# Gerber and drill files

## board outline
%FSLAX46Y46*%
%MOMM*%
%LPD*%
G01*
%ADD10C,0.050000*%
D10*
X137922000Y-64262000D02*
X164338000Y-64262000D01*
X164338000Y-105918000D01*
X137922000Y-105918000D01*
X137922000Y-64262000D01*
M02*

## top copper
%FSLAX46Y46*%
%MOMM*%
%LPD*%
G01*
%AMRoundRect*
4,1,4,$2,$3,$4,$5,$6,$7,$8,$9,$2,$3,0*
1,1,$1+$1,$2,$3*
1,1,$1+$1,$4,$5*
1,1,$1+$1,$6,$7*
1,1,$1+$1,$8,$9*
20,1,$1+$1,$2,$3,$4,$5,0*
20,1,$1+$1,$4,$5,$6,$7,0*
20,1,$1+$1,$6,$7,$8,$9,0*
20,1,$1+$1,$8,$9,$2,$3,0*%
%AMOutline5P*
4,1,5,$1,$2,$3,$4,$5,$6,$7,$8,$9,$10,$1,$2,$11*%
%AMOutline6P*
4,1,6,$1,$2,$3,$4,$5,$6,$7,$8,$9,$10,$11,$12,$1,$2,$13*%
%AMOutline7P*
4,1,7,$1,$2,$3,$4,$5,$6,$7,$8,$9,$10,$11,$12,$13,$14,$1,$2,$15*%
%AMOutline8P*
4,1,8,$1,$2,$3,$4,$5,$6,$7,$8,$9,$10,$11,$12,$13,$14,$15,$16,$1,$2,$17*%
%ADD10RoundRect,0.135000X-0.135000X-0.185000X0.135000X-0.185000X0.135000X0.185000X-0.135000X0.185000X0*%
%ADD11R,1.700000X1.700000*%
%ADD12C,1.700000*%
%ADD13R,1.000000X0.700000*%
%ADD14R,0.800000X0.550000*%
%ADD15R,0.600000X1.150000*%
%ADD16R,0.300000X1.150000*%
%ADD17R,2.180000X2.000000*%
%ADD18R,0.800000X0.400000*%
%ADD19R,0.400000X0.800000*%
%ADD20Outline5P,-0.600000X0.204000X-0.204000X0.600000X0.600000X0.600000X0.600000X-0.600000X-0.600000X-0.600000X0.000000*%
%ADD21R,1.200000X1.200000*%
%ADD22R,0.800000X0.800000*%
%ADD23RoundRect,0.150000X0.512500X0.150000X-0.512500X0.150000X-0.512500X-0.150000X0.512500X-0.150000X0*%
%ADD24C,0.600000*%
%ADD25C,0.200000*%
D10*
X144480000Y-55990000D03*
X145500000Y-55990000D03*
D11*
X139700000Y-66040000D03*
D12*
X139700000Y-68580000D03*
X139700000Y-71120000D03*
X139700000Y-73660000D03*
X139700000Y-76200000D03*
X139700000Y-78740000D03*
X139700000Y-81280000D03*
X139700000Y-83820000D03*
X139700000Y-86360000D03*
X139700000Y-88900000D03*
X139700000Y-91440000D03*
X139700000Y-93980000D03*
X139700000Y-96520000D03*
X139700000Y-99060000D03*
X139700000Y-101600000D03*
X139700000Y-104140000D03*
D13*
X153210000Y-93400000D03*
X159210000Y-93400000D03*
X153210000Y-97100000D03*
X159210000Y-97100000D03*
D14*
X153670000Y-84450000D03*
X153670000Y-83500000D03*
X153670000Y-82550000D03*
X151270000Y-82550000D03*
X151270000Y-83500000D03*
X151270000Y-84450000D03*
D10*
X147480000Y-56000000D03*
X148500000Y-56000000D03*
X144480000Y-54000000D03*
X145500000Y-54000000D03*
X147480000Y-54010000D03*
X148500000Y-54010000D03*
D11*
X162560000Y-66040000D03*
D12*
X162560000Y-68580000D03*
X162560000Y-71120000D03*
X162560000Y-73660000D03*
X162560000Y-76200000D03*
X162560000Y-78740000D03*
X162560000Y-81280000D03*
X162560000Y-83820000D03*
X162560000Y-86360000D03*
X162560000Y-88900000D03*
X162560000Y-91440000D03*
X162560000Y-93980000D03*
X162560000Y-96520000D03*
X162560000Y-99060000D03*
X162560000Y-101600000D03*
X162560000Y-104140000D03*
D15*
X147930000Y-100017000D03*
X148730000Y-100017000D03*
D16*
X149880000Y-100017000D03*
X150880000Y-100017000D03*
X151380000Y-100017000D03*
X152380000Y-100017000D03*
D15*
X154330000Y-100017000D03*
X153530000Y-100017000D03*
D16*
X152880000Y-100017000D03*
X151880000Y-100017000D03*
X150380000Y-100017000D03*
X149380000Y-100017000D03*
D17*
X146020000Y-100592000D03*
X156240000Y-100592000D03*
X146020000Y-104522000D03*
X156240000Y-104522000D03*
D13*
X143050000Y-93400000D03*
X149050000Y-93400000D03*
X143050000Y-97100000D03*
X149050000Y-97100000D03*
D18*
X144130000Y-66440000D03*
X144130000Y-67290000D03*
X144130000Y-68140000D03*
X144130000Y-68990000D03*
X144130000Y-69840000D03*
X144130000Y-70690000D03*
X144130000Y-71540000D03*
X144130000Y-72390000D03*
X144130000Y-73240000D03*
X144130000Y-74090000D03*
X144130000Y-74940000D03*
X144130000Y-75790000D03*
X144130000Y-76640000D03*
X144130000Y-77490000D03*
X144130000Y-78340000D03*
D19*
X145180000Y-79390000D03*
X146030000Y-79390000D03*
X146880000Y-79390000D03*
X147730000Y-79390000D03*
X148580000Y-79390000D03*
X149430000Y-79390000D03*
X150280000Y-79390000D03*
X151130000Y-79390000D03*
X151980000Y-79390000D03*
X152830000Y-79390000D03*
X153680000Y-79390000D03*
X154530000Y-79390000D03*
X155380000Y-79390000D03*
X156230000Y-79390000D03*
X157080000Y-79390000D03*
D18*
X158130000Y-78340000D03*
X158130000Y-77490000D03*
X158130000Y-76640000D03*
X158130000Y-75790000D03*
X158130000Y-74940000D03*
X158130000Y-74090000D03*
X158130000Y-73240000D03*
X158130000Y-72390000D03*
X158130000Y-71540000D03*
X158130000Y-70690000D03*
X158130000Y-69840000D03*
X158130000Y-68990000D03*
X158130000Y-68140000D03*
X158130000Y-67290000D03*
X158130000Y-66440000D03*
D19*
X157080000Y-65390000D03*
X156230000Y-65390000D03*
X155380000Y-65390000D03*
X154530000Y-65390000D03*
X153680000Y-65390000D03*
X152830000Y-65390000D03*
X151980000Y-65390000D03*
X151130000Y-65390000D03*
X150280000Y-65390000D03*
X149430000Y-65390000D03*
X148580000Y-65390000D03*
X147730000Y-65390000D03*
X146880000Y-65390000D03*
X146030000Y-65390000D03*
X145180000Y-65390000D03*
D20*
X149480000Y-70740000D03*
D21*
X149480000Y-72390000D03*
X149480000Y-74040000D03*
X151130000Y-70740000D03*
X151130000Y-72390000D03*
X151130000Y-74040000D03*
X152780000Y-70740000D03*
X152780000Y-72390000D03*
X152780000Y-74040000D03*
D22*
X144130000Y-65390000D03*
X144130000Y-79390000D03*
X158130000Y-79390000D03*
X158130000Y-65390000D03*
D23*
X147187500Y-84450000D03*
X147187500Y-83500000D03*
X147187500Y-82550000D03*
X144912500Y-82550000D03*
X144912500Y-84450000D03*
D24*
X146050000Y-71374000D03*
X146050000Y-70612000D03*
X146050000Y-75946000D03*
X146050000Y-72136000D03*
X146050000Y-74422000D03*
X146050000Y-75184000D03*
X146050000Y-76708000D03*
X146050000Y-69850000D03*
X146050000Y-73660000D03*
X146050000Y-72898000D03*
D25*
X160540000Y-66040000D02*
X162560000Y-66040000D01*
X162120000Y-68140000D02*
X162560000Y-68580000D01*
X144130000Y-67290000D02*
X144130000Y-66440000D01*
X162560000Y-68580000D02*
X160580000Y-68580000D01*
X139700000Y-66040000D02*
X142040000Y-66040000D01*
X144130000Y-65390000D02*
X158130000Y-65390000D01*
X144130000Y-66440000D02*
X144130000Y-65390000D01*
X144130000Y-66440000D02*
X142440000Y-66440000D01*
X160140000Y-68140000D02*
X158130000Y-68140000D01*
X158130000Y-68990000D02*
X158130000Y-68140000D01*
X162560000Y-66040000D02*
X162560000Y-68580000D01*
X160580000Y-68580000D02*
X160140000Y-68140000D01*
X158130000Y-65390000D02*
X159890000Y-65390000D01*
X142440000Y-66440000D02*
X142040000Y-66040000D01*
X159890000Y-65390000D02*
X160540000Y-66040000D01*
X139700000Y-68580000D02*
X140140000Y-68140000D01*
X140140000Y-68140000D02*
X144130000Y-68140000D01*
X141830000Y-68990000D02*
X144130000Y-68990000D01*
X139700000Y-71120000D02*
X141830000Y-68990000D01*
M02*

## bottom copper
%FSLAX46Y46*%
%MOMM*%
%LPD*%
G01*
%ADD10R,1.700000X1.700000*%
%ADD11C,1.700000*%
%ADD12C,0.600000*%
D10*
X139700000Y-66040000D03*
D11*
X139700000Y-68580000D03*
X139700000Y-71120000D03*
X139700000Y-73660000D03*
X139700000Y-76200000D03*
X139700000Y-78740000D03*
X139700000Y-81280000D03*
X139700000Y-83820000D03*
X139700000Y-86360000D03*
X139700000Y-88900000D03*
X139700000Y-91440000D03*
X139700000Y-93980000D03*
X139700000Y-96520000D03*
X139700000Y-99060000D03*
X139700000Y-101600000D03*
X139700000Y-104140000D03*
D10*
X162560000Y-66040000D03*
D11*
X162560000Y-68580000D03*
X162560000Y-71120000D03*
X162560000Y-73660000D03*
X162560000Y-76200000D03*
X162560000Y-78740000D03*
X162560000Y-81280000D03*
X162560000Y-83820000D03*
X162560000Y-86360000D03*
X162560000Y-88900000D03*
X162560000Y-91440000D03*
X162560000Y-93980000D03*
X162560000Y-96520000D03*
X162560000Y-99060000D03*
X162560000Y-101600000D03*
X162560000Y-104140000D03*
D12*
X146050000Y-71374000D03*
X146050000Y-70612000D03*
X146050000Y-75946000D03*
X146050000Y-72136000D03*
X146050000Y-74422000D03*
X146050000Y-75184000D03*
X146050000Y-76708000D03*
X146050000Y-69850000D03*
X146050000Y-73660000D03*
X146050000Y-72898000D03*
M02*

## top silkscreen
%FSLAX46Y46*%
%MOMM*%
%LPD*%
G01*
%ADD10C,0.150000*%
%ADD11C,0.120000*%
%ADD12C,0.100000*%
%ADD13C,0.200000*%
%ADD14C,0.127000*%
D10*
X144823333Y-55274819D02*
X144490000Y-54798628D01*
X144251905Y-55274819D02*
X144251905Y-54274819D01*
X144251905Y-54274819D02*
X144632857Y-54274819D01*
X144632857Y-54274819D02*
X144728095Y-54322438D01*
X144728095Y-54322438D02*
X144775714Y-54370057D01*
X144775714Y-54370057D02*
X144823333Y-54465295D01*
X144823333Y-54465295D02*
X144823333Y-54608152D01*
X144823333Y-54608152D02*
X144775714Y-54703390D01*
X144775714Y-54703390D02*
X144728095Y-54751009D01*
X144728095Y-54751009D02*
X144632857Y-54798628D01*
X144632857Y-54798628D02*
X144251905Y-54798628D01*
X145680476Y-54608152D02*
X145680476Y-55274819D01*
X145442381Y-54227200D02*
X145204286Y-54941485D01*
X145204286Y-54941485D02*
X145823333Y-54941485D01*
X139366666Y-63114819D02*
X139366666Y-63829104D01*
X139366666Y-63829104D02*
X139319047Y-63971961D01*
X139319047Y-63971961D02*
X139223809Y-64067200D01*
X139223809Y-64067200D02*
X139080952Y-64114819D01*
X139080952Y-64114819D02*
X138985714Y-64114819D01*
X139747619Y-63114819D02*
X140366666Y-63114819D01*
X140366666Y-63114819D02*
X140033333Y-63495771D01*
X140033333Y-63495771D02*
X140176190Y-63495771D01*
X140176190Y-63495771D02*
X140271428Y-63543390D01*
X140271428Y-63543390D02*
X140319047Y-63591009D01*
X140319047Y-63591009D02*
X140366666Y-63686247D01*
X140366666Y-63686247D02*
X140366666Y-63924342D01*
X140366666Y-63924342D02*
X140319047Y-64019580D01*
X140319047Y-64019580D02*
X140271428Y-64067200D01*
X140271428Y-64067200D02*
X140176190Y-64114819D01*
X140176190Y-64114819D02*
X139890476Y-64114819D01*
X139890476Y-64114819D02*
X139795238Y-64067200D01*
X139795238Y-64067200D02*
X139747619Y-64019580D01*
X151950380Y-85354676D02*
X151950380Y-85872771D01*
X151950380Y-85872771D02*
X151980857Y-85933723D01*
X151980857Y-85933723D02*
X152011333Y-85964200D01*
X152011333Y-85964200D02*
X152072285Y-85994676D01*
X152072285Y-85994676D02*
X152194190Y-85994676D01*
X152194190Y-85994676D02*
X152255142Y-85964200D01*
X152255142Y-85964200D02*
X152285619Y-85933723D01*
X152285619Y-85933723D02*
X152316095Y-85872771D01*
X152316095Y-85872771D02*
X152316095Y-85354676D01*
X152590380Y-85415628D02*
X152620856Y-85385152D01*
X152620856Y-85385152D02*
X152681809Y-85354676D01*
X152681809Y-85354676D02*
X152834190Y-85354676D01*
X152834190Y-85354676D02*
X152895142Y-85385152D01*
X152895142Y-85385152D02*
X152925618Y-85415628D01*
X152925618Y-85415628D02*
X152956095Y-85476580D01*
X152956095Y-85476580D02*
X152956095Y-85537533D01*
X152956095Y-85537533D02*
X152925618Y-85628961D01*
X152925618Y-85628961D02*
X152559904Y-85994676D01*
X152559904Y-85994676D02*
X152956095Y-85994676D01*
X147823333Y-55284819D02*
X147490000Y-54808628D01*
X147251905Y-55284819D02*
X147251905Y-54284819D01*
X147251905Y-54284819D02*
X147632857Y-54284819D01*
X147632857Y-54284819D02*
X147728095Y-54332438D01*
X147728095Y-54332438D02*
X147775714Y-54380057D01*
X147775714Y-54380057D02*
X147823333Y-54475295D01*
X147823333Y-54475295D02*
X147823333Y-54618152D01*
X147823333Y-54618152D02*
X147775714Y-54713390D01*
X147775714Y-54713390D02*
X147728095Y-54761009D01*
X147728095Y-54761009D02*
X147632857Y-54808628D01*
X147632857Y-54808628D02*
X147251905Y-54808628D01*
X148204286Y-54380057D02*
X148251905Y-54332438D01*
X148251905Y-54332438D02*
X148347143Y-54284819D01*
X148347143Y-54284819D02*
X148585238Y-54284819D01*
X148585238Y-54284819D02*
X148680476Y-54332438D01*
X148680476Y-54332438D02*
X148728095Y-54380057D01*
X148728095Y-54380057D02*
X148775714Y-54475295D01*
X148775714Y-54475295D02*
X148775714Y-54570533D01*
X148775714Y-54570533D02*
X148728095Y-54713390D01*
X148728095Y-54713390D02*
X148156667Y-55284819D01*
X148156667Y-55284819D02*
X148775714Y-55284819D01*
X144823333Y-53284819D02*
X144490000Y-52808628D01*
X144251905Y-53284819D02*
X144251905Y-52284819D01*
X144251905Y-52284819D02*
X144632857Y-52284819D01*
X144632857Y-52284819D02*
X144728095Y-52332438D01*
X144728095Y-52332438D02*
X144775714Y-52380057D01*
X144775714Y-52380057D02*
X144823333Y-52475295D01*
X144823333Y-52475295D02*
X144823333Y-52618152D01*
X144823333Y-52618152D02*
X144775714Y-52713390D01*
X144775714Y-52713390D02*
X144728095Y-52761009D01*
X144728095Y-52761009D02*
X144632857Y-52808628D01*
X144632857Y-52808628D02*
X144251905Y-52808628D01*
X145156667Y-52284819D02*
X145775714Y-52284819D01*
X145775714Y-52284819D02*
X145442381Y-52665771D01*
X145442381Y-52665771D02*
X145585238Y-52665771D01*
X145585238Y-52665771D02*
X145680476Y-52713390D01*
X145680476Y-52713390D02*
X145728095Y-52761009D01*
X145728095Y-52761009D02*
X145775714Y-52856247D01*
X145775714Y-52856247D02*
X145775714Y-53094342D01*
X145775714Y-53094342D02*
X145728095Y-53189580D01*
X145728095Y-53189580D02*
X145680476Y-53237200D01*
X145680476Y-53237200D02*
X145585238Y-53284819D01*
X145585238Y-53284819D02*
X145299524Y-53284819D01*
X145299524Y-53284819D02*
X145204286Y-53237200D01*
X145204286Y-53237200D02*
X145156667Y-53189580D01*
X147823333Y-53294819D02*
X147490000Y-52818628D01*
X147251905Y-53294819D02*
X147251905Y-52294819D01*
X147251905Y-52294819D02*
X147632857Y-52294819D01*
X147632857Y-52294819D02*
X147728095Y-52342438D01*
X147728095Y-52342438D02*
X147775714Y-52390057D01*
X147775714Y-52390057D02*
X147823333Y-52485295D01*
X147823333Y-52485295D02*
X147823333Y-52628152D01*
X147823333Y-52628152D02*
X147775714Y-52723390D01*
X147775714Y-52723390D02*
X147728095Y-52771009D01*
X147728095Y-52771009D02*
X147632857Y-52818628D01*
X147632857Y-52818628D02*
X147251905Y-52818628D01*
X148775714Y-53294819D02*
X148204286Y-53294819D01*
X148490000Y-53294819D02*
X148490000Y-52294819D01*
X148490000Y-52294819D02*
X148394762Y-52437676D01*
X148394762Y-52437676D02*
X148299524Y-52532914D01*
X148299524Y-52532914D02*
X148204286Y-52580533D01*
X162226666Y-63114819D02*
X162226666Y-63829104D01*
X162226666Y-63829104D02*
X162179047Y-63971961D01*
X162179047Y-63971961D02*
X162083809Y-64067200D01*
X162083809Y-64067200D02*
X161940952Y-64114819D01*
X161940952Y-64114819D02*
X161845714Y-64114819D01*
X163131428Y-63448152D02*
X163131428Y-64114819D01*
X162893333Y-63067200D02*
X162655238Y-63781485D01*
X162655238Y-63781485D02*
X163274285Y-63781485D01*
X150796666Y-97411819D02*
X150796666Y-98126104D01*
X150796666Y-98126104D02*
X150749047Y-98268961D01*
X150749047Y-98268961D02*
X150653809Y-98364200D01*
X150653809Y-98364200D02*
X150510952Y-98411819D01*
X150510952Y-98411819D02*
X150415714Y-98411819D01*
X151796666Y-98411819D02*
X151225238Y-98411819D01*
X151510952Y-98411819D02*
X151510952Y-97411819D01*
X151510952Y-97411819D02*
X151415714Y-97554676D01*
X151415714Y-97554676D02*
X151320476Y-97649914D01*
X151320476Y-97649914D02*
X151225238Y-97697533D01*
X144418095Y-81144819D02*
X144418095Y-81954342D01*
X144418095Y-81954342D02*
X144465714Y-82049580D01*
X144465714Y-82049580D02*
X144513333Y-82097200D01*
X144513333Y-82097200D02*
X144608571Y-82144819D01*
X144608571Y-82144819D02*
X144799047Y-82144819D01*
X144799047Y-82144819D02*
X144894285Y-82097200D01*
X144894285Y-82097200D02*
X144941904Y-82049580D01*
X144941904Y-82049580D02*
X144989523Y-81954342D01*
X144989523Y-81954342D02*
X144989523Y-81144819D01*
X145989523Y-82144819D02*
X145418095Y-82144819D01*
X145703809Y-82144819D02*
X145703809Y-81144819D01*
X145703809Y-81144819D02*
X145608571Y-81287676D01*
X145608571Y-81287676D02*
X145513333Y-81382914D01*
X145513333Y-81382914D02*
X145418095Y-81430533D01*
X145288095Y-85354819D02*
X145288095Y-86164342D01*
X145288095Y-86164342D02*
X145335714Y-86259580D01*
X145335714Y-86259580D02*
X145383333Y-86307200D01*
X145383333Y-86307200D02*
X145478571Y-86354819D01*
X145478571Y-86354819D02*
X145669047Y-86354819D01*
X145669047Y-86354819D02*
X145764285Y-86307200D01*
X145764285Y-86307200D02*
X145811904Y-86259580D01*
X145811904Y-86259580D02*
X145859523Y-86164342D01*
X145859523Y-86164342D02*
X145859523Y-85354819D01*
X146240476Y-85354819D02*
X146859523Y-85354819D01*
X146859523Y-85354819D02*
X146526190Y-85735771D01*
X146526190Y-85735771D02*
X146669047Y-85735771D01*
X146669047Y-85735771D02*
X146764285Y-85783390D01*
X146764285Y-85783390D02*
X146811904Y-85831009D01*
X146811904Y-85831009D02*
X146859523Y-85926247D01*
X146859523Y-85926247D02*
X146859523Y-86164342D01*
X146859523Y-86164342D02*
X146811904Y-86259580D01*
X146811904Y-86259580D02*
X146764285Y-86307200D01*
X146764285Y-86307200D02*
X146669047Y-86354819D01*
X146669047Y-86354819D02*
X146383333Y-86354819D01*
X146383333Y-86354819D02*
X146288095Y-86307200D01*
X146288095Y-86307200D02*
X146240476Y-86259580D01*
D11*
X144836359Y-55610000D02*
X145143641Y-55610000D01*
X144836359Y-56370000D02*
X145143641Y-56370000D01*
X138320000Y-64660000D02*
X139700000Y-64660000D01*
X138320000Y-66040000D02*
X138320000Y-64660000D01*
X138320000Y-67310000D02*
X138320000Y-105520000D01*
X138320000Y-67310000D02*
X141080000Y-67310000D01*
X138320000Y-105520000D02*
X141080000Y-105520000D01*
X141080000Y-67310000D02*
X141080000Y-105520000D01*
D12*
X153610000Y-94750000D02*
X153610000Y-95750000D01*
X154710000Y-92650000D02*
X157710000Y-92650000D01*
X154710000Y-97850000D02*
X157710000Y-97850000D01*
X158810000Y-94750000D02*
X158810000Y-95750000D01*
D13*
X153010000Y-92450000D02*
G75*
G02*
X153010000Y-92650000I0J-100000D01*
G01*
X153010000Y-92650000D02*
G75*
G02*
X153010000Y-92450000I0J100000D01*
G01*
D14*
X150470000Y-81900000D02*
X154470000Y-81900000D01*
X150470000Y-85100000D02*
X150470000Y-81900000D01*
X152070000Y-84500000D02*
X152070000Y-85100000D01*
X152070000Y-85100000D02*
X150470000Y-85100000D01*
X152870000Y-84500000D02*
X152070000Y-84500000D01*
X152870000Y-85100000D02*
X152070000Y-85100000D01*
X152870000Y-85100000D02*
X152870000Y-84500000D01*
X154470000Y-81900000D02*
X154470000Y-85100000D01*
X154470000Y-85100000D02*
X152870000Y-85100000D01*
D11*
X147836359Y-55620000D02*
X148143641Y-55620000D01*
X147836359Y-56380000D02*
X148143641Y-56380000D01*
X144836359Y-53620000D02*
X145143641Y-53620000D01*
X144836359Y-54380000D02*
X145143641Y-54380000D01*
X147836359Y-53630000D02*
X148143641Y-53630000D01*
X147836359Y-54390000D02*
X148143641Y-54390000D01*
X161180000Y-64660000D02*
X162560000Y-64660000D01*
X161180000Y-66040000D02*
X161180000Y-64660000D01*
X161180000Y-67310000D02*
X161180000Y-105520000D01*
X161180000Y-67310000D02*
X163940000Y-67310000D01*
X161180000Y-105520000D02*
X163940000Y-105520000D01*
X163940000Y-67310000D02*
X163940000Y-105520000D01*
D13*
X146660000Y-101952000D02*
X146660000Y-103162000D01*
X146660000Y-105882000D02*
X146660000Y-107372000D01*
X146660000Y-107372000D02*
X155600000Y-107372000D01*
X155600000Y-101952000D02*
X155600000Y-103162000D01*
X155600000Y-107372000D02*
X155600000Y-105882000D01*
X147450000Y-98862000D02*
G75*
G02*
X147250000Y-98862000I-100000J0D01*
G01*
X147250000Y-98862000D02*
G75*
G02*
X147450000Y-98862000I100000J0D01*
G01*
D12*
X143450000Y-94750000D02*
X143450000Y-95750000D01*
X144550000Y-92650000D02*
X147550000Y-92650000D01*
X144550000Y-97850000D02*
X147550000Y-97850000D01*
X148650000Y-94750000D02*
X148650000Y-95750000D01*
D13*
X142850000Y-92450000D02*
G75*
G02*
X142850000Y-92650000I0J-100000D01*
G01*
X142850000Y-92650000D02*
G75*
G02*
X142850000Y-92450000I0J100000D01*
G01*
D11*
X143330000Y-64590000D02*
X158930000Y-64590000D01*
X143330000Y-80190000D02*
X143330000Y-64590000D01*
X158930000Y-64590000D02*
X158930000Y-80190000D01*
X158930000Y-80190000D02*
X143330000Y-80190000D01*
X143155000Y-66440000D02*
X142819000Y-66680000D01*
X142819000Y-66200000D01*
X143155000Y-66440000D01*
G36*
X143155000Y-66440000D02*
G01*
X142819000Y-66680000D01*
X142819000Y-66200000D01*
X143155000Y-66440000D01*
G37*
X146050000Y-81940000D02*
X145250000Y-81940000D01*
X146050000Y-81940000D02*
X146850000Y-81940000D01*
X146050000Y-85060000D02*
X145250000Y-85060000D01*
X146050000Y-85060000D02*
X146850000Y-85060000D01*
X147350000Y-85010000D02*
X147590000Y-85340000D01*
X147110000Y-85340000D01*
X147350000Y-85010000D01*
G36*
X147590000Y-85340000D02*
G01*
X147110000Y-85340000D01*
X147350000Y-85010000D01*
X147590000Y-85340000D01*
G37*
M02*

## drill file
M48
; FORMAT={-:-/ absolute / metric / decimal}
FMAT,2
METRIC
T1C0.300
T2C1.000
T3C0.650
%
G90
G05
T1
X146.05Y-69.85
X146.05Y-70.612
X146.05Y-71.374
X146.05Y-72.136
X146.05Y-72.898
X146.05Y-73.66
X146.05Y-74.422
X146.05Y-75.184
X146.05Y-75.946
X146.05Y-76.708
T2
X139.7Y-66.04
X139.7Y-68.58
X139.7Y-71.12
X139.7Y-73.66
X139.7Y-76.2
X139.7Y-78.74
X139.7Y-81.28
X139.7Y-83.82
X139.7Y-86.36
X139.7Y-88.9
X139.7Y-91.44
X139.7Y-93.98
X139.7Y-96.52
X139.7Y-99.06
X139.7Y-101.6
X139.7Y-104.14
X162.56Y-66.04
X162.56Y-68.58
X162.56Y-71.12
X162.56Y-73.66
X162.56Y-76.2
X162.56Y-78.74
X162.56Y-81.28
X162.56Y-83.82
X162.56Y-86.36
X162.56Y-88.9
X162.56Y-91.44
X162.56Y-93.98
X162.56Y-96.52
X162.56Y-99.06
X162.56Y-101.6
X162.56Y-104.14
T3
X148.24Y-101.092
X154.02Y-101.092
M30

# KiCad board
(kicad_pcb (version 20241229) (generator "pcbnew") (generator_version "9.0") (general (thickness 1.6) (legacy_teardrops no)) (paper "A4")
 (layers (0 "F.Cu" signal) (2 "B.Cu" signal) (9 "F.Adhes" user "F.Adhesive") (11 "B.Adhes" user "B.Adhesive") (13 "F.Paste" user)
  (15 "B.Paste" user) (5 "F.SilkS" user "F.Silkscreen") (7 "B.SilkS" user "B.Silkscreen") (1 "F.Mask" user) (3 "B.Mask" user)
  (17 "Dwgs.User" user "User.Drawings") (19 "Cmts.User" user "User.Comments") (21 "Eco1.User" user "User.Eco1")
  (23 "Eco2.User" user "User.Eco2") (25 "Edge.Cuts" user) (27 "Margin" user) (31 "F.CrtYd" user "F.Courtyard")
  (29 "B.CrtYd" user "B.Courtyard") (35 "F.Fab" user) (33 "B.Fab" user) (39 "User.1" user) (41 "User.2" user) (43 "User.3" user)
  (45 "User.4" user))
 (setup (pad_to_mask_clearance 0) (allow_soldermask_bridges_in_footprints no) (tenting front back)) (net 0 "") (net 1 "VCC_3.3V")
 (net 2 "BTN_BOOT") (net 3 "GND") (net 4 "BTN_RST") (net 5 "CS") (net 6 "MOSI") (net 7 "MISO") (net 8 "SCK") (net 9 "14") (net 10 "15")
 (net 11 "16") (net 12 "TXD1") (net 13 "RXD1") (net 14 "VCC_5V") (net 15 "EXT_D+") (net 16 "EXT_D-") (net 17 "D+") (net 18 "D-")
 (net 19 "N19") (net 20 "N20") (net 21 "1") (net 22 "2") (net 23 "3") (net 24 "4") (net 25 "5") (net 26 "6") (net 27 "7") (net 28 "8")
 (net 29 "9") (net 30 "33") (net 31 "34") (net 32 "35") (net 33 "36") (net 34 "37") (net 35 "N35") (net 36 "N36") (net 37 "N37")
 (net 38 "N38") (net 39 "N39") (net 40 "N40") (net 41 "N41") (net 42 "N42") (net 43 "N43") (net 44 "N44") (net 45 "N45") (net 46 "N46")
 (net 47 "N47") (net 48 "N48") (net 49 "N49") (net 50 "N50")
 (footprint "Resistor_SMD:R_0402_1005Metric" (layer "F.Cu") (at 144.99 55.99)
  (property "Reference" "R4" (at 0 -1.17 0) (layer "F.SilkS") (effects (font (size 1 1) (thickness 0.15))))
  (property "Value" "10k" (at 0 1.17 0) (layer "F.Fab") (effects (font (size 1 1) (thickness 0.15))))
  (fp_line (start -0.153641 -0.38) (end 0.153641 -0.38) (stroke (width 0.12) (type solid)) (layer "F.SilkS"))
  (fp_line (start -0.153641 0.38) (end 0.153641 0.38) (stroke (width 0.12) (type solid)) (layer "F.SilkS"))
  (pad "1" smd roundrect (at -0.51 0) (size 0.54 0.64) (layers "F.Cu" "F.Mask" "F.Paste") (roundrect_rratio 0.25) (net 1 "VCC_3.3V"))
  (pad "2" smd roundrect (at 0.51 0) (size 0.54 0.64) (layers "F.Cu" "F.Mask" "F.Paste") (roundrect_rratio 0.25) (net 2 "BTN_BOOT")))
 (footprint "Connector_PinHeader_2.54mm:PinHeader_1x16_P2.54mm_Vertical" (layer "F.Cu") (at 139.7 66.04)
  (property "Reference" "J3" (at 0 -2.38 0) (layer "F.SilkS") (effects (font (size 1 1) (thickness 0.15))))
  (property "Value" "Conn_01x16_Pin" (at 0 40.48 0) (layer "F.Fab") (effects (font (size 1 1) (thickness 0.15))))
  (fp_line (start -1.38 -1.38) (end 0 -1.38) (stroke (width 0.12) (type solid)) (layer "F.SilkS"))
  (fp_line (start -1.38 0) (end -1.38 -1.38) (stroke (width 0.12) (type solid)) (layer "F.SilkS"))
  (fp_line (start -1.38 1.27) (end -1.38 39.48) (stroke (width 0.12) (type solid)) (layer "F.SilkS"))
  (fp_line (start -1.38 1.27) (end 1.38 1.27) (stroke (width 0.12) (type solid)) (layer "F.SilkS"))
  (fp_line (start -1.38 39.48) (end 1.38 39.48) (stroke (width 0.12) (type solid)) (layer "F.SilkS"))
  (fp_line (start 1.38 1.27) (end 1.38 39.48) (stroke (width 0.12) (type solid)) (layer "F.SilkS"))
  (pad "1" thru_hole rect (at 0 0) (size 1.7 1.7) (drill 1) (layers "*.Cu" "*.Mask") (remove_unused_layers no) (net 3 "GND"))
  (pad "2" thru_hole circle (at 0 2.54) (size 1.7 1.7) (drill 1) (layers "*.Cu" "*.Mask") (remove_unused_layers no) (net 1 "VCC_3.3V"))
  (pad "3" thru_hole circle (at 0 5.08) (size 1.7 1.7) (drill 1) (layers "*.Cu" "*.Mask") (remove_unused_layers no) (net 2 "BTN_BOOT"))
  (pad "4" thru_hole circle (at 0 7.62) (size 1.7 1.7) (drill 1) (layers "*.Cu" "*.Mask") (remove_unused_layers no) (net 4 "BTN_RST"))
  (pad "5" thru_hole circle (at 0 10.16) (size 1.7 1.7) (drill 1) (layers "*.Cu" "*.Mask") (remove_unused_layers no) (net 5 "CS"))
  (pad "6" thru_hole circle (at 0 12.7) (size 1.7 1.7) (drill 1) (layers "*.Cu" "*.Mask") (remove_unused_layers no) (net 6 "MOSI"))
  (pad "7" thru_hole circle (at 0 15.24) (size 1.7 1.7) (drill 1) (layers "*.Cu" "*.Mask") (remove_unused_layers no) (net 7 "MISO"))
  (pad "8" thru_hole circle (at 0 17.78) (size 1.7 1.7) (drill 1) (layers "*.Cu" "*.Mask") (remove_unused_layers no) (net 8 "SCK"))
  (pad "9" thru_hole circle (at 0 20.32) (size 1.7 1.7) (drill 1) (layers "*.Cu" "*.Mask") (remove_unused_layers no) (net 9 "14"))
  (pad "10" thru_hole circle (at 0 22.86) (size 1.7 1.7) (drill 1) (layers "*.Cu" "*.Mask") (remove_unused_layers no) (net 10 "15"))
  (pad "11" thru_hole circle (at 0 25.4) (size 1.7 1.7) (drill 1) (layers "*.Cu" "*.Mask") (remove_unused_layers no) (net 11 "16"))
  (pad "12" thru_hole circle (at 0 27.94) (size 1.7 1.7) (drill 1) (layers "*.Cu" "*.Mask") (remove_unused_layers no) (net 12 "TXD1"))
  (pad "13" thru_hole circle (at 0 30.48) (size 1.7 1.7) (drill 1) (layers "*.Cu" "*.Mask") (remove_unused_layers no) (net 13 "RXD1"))
  (pad "14" thru_hole circle (at 0 33.02) (size 1.7 1.7) (drill 1) (layers "*.Cu" "*.Mask") (remove_unused_layers no) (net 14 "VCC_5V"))
  (pad "15" thru_hole circle (at 0 35.56) (size 1.7 1.7) (drill 1) (layers "*.Cu" "*.Mask") (remove_unused_layers no) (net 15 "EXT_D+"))
  (pad "16" thru_hole circle (at 0 38.1) (size 1.7 1.7) (drill 1) (layers "*.Cu" "*.Mask") (remove_unused_layers no) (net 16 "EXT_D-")))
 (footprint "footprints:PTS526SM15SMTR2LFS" (layer "F.Cu") (at 156.21 95.25)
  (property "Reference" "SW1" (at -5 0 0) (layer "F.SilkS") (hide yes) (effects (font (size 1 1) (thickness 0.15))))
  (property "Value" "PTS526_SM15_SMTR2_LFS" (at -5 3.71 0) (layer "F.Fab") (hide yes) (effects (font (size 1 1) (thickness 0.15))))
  (fp_line (start -2.6 -0.5) (end -2.6 0.5) (stroke (width 0.1) (type solid)) (layer "F.SilkS"))
  (fp_line (start -1.5 -2.6) (end 1.5 -2.6) (stroke (width 0.1) (type solid)) (layer "F.SilkS"))
  (fp_line (start -1.5 2.6) (end 1.5 2.6) (stroke (width 0.1) (type solid)) (layer "F.SilkS"))
  (fp_line (start 2.6 -0.5) (end 2.6 0.5) (stroke (width 0.1) (type solid)) (layer "F.SilkS"))
  (fp_arc (start -3.2 -2.8) (mid -3.1 -2.7) (end -3.2 -2.6) (stroke (width 0.2) (type solid)) (layer "F.SilkS"))
  (fp_arc (start -3.2 -2.6) (mid -3.3 -2.7) (end -3.2 -2.8) (stroke (width 0.2) (type solid)) (layer "F.SilkS"))
  (pad "1" smd rect (at -3 -1.85) (size 1 0.7) (layers "F.Cu" "F.Mask" "F.Paste") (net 3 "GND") (solder_mask_margin 0.102))
  (pad "2" smd rect (at 3 -1.85) (size 1 0.7) (layers "F.Cu" "F.Mask" "F.Paste") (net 3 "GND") (solder_mask_margin 0.102))
  (pad "3" smd rect (at -3 1.85) (size 1 0.7) (layers "F.Cu" "F.Mask" "F.Paste") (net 4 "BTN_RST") (solder_mask_margin 0.102))
  (pad "4" smd rect (at 3 1.85) (size 1 0.7) (layers "F.Cu" "F.Mask" "F.Paste") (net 4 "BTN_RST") (solder_mask_margin 0.102)))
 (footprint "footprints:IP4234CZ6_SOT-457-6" (layer "F.Cu") (at 152.47 83.5 180)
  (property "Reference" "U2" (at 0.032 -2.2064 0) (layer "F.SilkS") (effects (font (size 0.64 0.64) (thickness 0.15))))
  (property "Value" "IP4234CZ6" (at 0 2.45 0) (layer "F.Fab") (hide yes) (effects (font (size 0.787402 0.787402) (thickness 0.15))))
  (fp_line (start 2 1.6) (end -2 1.6) (stroke (width 0.127) (type solid)) (layer "F.SilkS"))
  (fp_line (start 2 -1.6) (end 2 1.6) (stroke (width 0.127) (type solid)) (layer "F.SilkS"))
  (fp_line (start 0.4 -1) (end 0.4 -1.6) (stroke (width 0.127) (type solid)) (layer "F.SilkS"))
  (fp_line (start 0.4 -1.6) (end 2 -1.6) (stroke (width 0.127) (type solid)) (layer "F.SilkS"))
  (fp_line (start -0.4 -1) (end 0.4 -1) (stroke (width 0.127) (type solid)) (layer "F.SilkS"))
  (fp_line (start -0.4 -1.6) (end 0.4 -1.6) (stroke (width 0.127) (type solid)) (layer "F.SilkS"))
  (fp_line (start -0.4 -1.6) (end -0.4 -1) (stroke (width 0.127) (type solid)) (layer "F.SilkS"))
  (fp_line (start -2 1.6) (end -2 -1.6) (stroke (width 0.127) (type solid)) (layer "F.SilkS"))
  (fp_line (start -2 -1.6) (end -0.4 -1.6) (stroke (width 0.127) (type solid)) (layer "F.SilkS"))
  (pad "1" smd rect (at -1.2 -0.95 180) (size 0.8 0.55) (layers "F.Cu" "F.Mask" "F.Paste") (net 15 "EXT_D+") (solder_mask_margin 0.102))
  (pad "2" smd rect (at -1.2 0 180) (size 0.8 0.55) (layers "F.Cu" "F.Mask" "F.Paste") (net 3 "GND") (solder_mask_margin 0.102))
  (pad "3" smd rect (at -1.2 0.95 180) (size 0.8 0.55) (layers "F.Cu" "F.Mask" "F.Paste") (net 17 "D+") (solder_mask_margin 0.102))
  (pad "4" smd rect (at 1.2 0.95 180) (size 0.8 0.55) (layers "F.Cu" "F.Mask" "F.Paste") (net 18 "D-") (solder_mask_margin 0.102))
  (pad "5" smd rect (at 1.2 0 180) (size 0.8 0.55) (layers "F.Cu" "F.Mask" "F.Paste") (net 14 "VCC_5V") (solder_mask_margin 0.102))
  (pad "6" smd rect (at 1.2 -0.95 180) (size 0.8 0.55) (layers "F.Cu" "F.Mask" "F.Paste") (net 16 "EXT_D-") (solder_mask_margin 0.102)))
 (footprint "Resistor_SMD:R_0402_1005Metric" (layer "F.Cu") (at 147.99 56)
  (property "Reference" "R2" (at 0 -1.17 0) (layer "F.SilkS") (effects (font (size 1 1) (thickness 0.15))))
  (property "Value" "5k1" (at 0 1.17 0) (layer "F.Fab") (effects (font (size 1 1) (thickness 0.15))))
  (fp_line (start -0.153641 -0.38) (end 0.153641 -0.38) (stroke (width 0.12) (type solid)) (layer "F.SilkS"))
  (fp_line (start -0.153641 0.38) (end 0.153641 0.38) (stroke (width 0.12) (type solid)) (layer "F.SilkS"))
  (pad "1" smd roundrect (at -0.51 0) (size 0.54 0.64) (layers "F.Cu" "F.Mask" "F.Paste") (roundrect_rratio 0.25) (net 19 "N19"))
  (pad "2" smd roundrect (at 0.51 0) (size 0.54 0.64) (layers "F.Cu" "F.Mask" "F.Paste") (roundrect_rratio 0.25) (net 3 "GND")))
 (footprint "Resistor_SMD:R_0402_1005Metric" (layer "F.Cu") (at 144.99 54)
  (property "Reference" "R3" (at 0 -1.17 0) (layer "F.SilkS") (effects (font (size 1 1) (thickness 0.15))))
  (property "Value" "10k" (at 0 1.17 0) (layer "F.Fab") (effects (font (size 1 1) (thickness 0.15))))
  (fp_line (start -0.153641 -0.38) (end 0.153641 -0.38) (stroke (width 0.12) (type solid)) (layer "F.SilkS"))
  (fp_line (start -0.153641 0.38) (end 0.153641 0.38) (stroke (width 0.12) (type solid)) (layer "F.SilkS"))
  (pad "1" smd roundrect (at -0.51 0) (size 0.54 0.64) (layers "F.Cu" "F.Mask" "F.Paste") (roundrect_rratio 0.25) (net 1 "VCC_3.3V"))
  (pad "2" smd roundrect (at 0.51 0) (size 0.54 0.64) (layers "F.Cu" "F.Mask" "F.Paste") (roundrect_rratio 0.25) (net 4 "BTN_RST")))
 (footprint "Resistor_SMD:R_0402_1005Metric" (layer "F.Cu") (at 147.99 54.01)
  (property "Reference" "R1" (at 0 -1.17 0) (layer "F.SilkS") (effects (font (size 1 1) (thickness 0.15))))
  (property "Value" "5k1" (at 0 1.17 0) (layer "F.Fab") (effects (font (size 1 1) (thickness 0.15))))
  (fp_line (start -0.153641 -0.38) (end 0.153641 -0.38) (stroke (width 0.12) (type solid)) (layer "F.SilkS"))
  (fp_line (start -0.153641 0.38) (end 0.153641 0.38) (stroke (width 0.12) (type solid)) (layer "F.SilkS"))
  (pad "1" smd roundrect (at -0.51 0) (size 0.54 0.64) (layers "F.Cu" "F.Mask" "F.Paste") (roundrect_rratio 0.25) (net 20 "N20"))
  (pad "2" smd roundrect (at 0.51 0) (size 0.54 0.64) (layers "F.Cu" "F.Mask" "F.Paste") (roundrect_rratio 0.25) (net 3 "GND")))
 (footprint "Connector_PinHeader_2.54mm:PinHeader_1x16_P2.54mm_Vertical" (layer "F.Cu") (at 162.56 66.04)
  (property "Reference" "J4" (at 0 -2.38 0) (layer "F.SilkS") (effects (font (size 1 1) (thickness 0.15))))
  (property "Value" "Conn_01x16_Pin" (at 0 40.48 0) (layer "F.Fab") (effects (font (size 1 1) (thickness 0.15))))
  (fp_line (start -1.38 -1.38) (end 0 -1.38) (stroke (width 0.12) (type solid)) (layer "F.SilkS"))
  (fp_line (start -1.38 0) (end -1.38 -1.38) (stroke (width 0.12) (type solid)) (layer "F.SilkS"))
  (fp_line (start -1.38 1.27) (end -1.38 39.48) (stroke (width 0.12) (type solid)) (layer "F.SilkS"))
  (fp_line (start -1.38 1.27) (end 1.38 1.27) (stroke (width 0.12) (type solid)) (layer "F.SilkS"))
  (fp_line (start -1.38 39.48) (end 1.38 39.48) (stroke (width 0.12) (type solid)) (layer "F.SilkS"))
  (fp_line (start 1.38 1.27) (end 1.38 39.48) (stroke (width 0.12) (type solid)) (layer "F.SilkS"))
  (pad "1" thru_hole rect (at 0 0) (size 1.7 1.7) (drill 1) (layers "*.Cu" "*.Mask") (remove_unused_layers no) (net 3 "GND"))
  (pad "2" thru_hole circle (at 0 2.54) (size 1.7 1.7) (drill 1) (layers "*.Cu" "*.Mask") (remove_unused_layers no) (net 3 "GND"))
  (pad "3" thru_hole circle (at 0 5.08) (size 1.7 1.7) (drill 1) (layers "*.Cu" "*.Mask") (remove_unused_layers no) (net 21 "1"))
  (pad "4" thru_hole circle (at 0 7.62) (size 1.7 1.7) (drill 1) (layers "*.Cu" "*.Mask") (remove_unused_layers no) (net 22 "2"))
  (pad "5" thru_hole circle (at 0 10.16) (size 1.7 1.7) (drill 1) (layers "*.Cu" "*.Mask") (remove_unused_layers no) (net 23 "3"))
  (pad "6" thru_hole circle (at 0 12.7) (size 1.7 1.7) (drill 1) (layers "*.Cu" "*.Mask") (remove_unused_layers no) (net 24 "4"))
  (pad "7" thru_hole circle (at 0 15.24) (size 1.7 1.7) (drill 1) (layers "*.Cu" "*.Mask") (remove_unused_layers no) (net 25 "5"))
  (pad "8" thru_hole circle (at 0 17.78) (size 1.7 1.7) (drill 1) (layers "*.Cu" "*.Mask") (remove_unused_layers no) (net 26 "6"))
  (pad "9" thru_hole circle (at 0 20.32) (size 1.7 1.7) (drill 1) (layers "*.Cu" "*.Mask") (remove_unused_layers no) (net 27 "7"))
  (pad "10" thru_hole circle (at 0 22.86) (size 1.7 1.7) (drill 1) (layers "*.Cu" "*.Mask") (remove_unused_layers no) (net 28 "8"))
  (pad "11" thru_hole circle (at 0 25.4) (size 1.7 1.7) (drill 1) (layers "*.Cu" "*.Mask") (remove_unused_layers no) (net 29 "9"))
  (pad "12" thru_hole circle (at 0 27.94) (size 1.7 1.7) (drill 1) (layers "*.Cu" "*.Mask") (remove_unused_layers no) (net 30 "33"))
  (pad "13" thru_hole circle (at 0 30.48) (size 1.7 1.7) (drill 1) (layers "*.Cu" "*.Mask") (remove_unused_layers no) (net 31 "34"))
  (pad "14" thru_hole circle (at 0 33.02) (size 1.7 1.7) (drill 1) (layers "*.Cu" "*.Mask") (remove_unused_layers no) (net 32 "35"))
  (pad "15" thru_hole circle (at 0 35.56) (size 1.7 1.7) (drill 1) (layers "*.Cu" "*.Mask") (remove_unused_layers no) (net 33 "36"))
  (pad "16" thru_hole circle (at 0 38.1) (size 1.7 1.7) (drill 1) (layers "*.Cu" "*.Mask") (remove_unused_layers no) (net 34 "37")))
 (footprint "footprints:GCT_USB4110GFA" (layer "F.Cu") (at 151.13 101.092)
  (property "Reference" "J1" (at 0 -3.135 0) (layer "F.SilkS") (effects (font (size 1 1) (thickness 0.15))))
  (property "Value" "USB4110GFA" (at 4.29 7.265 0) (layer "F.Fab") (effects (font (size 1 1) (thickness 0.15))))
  (fp_line (start -4.47 0.86) (end -4.47 2.07) (stroke (width 0.2) (type solid)) (layer "F.SilkS"))
  (fp_line (start -4.47 4.79) (end -4.47 6.28) (stroke (width 0.2) (type solid)) (layer "F.SilkS"))
  (fp_line (start -4.47 6.28) (end 4.47 6.28) (stroke (width 0.2) (type solid)) (layer "F.SilkS"))
  (fp_line (start 4.47 0.86) (end 4.47 2.07) (stroke (width 0.2) (type solid)) (layer "F.SilkS"))
  (fp_line (start 4.47 6.28) (end 4.47 4.79) (stroke (width 0.2) (type solid)) (layer "F.SilkS"))
  (fp_circle (center -3.78 -2.23) (end -3.68 -2.23) (stroke (width 0.2) (type solid)) (fill no) (layer "F.SilkS"))
  (pad "" np_thru_hole circle (at -2.89 0) (size 0.65 0.65) (drill 0.65) (layers "*.Cu" "*.Mask"))
  (pad "" np_thru_hole circle (at 2.89 0) (size 0.65 0.65) (drill 0.65) (layers "*.Cu" "*.Mask"))
  (pad "A1/B12" smd rect (at -3.2 -1.075) (size 0.6 1.15) (layers "F.Cu" "F.Mask" "F.Paste") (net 3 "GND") (solder_mask_margin 0.102))
  (pad "A4/B9" smd rect (at -2.4 -1.075) (size 0.6 1.15) (layers "F.Cu" "F.Mask" "F.Paste") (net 14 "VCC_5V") (solder_mask_margin 0.102))
  (pad "A5" smd rect (at -1.25 -1.075) (size 0.3 1.15) (layers "F.Cu" "F.Mask" "F.Paste") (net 20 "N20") (solder_mask_margin 0.102))
  (pad "A6" smd rect (at -0.25 -1.075) (size 0.3 1.15) (layers "F.Cu" "F.Mask" "F.Paste") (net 15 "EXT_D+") (solder_mask_margin 0.102))
  (pad "A7" smd rect (at 0.25 -1.075) (size 0.3 1.15) (layers "F.Cu" "F.Mask" "F.Paste") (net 16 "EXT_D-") (solder_mask_margin 0.102))
  (pad "A8" smd rect (at 1.25 -1.075) (size 0.3 1.15) (layers "F.Cu" "F.Mask" "F.Paste") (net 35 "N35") (solder_mask_margin 0.102))
  (pad "B1/A12" smd rect (at 3.2 -1.075) (size 0.6 1.15) (layers "F.Cu" "F.Mask" "F.Paste") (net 3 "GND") (solder_mask_margin 0.102))
  (pad "B4/A9" smd rect (at 2.4 -1.075) (size 0.6 1.15) (layers "F.Cu" "F.Mask" "F.Paste") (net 14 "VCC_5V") (solder_mask_margin 0.102))
  (pad "B5" smd rect (at 1.75 -1.075) (size 0.3 1.15) (layers "F.Cu" "F.Mask" "F.Paste") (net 19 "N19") (solder_mask_margin 0.102))
  (pad "B6" smd rect (at 0.75 -1.075) (size 0.3 1.15) (layers "F.Cu" "F.Mask" "F.Paste") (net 15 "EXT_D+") (solder_mask_margin 0.102))
  (pad "B7" smd rect (at -0.75 -1.075) (size 0.3 1.15) (layers "F.Cu" "F.Mask" "F.Paste") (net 16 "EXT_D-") (solder_mask_margin 0.102))
  (pad "B8" smd rect (at -1.75 -1.075) (size 0.3 1.15) (layers "F.Cu" "F.Mask" "F.Paste") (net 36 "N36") (solder_mask_margin 0.102))
  (pad "S1" smd rect (at -5.11 -0.5) (size 2.18 2) (layers "F.Cu" "F.Mask" "F.Paste") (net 3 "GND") (solder_mask_margin 0.102))
  (pad "S2" smd rect (at 5.11 -0.5) (size 2.18 2) (layers "F.Cu" "F.Mask" "F.Paste") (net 3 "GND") (solder_mask_margin 0.102))
  (pad "S3" smd rect (at -5.11 3.43) (size 2.18 2) (layers "F.Cu" "F.Mask" "F.Paste") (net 3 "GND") (solder_mask_margin 0.102))
  (pad "S4" smd rect (at 5.11 3.43) (size 2.18 2) (layers "F.Cu" "F.Mask" "F.Paste") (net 3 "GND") (solder_mask_margin 0.102)))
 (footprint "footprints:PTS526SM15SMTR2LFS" (layer "F.Cu") (at 146.05 95.25)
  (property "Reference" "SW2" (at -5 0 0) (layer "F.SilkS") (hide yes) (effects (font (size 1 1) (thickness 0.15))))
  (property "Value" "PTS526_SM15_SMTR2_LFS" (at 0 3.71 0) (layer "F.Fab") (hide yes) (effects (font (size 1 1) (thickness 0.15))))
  (fp_line (start -2.6 -0.5) (end -2.6 0.5) (stroke (width 0.1) (type solid)) (layer "F.SilkS"))
  (fp_line (start -1.5 -2.6) (end 1.5 -2.6) (stroke (width 0.1) (type solid)) (layer "F.SilkS"))
  (fp_line (start -1.5 2.6) (end 1.5 2.6) (stroke (width 0.1) (type solid)) (layer "F.SilkS"))
  (fp_line (start 2.6 -0.5) (end 2.6 0.5) (stroke (width 0.1) (type solid)) (layer "F.SilkS"))
  (fp_arc (start -3.2 -2.8) (mid -3.1 -2.7) (end -3.2 -2.6) (stroke (width 0.2) (type solid)) (layer "F.SilkS"))
  (fp_arc (start -3.2 -2.6) (mid -3.3 -2.7) (end -3.2 -2.8) (stroke (width 0.2) (type solid)) (layer "F.SilkS"))
  (pad "1" smd rect (at -3 -1.85) (size 1 0.7) (layers "F.Cu" "F.Mask" "F.Paste") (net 3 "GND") (solder_mask_margin 0.102))
  (pad "2" smd rect (at 3 -1.85) (size 1 0.7) (layers "F.Cu" "F.Mask" "F.Paste") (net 3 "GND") (solder_mask_margin 0.102))
  (pad "3" smd rect (at -3 1.85) (size 1 0.7) (layers "F.Cu" "F.Mask" "F.Paste") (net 2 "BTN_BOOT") (solder_mask_margin 0.102))
  (pad "4" smd rect (at 3 1.85) (size 1 0.7) (layers "F.Cu" "F.Mask" "F.Paste") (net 2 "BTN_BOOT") (solder_mask_margin 0.102)))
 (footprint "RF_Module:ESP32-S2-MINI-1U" (layer "F.Cu") (at 151.13 72.39)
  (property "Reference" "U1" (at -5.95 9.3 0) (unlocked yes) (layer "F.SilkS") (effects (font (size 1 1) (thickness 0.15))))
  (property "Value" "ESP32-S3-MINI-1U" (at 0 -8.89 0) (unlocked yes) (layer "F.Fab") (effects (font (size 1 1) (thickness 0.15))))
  (fp_line (start -7.8 -7.8) (end 7.8 -7.8) (stroke (width 0.12) (type solid)) (layer "F.SilkS"))
  (fp_line (start -7.8 7.8) (end -7.8 -7.8) (stroke (width 0.12) (type solid)) (layer "F.SilkS"))
  (fp_line (start 7.8 -7.8) (end 7.8 7.8) (stroke (width 0.12) (type solid)) (layer "F.SilkS"))
  (fp_line (start 7.8 7.8) (end -7.8 7.8) (stroke (width 0.12) (type solid)) (layer "F.SilkS"))
  (fp_poly
   (pts (xy -7.975 -5.95) (xy -8.311 -5.71) (xy -8.311 -6.19) (xy -7.975 -5.95)) (stroke (width 0.12) (type solid)) (fill yes)
   (layer "F.SilkS"))
  (pad "1" smd rect (at -7 -5.95) (size 0.8 0.4) (layers "F.Cu" "F.Mask" "F.Paste") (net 3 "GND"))
  (pad "2" smd rect (at -7 -5.1) (size 0.8 0.4) (layers "F.Cu" "F.Mask" "F.Paste") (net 3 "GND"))
  (pad "3" smd rect (at -7 -4.25) (size 0.8 0.4) (layers "F.Cu" "F.Mask" "F.Paste") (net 1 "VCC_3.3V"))
  (pad "4" smd rect (at -7 -3.4) (size 0.8 0.4) (layers "F.Cu" "F.Mask" "F.Paste") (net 2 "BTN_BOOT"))
  (pad "5" smd rect (at -7 -2.55) (size 0.8 0.4) (layers "F.Cu" "F.Mask" "F.Paste") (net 21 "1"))
  (pad "6" smd rect (at -7 -1.7) (size 0.8 0.4) (layers "F.Cu" "F.Mask" "F.Paste") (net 22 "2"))
  (pad "7" smd rect (at -7 -0.85) (size 0.8 0.4) (layers "F.Cu" "F.Mask" "F.Paste") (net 23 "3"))
  (pad "8" smd rect (at -7 0) (size 0.8 0.4) (layers "F.Cu" "F.Mask" "F.Paste") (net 24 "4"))
  (pad "9" smd rect (at -7 0.85) (size 0.8 0.4) (layers "F.Cu" "F.Mask" "F.Paste") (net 25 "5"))
  (pad "10" smd rect (at -7 1.7) (size 0.8 0.4) (layers "F.Cu" "F.Mask" "F.Paste") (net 26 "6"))
  (pad "11" smd rect (at -7 2.55) (size 0.8 0.4) (layers "F.Cu" "F.Mask" "F.Paste") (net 27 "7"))
  (pad "12" smd rect (at -7 3.4) (size 0.8 0.4) (layers "F.Cu" "F.Mask" "F.Paste") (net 28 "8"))
  (pad "13" smd rect (at -7 4.25) (size 0.8 0.4) (layers "F.Cu" "F.Mask" "F.Paste") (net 29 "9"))
  (pad "14" smd rect (at -7 5.1) (size 0.8 0.4) (layers "F.Cu" "F.Mask" "F.Paste") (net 5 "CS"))
  (pad "15" smd rect (at -7 5.95) (size 0.8 0.4) (layers "F.Cu" "F.Mask" "F.Paste") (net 6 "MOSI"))
  (pad "16" smd rect (at -5.95 7 90) (size 0.8 0.4) (layers "F.Cu" "F.Mask" "F.Paste") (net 7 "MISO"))
  (pad "17" smd rect (at -5.1 7 90) (size 0.8 0.4) (layers "F.Cu" "F.Mask" "F.Paste") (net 8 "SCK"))
  (pad "18" smd rect (at -4.25 7 90) (size 0.8 0.4) (layers "F.Cu" "F.Mask" "F.Paste") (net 9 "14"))
  (pad "19" smd rect (at -3.4 7 90) (size 0.8 0.4) (layers "F.Cu" "F.Mask" "F.Paste") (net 10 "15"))
  (pad "20" smd rect (at -2.55 7 90) (size 0.8 0.4) (layers "F.Cu" "F.Mask" "F.Paste") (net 11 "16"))
  (pad "21" smd rect (at -1.7 7 90) (size 0.8 0.4) (layers "F.Cu" "F.Mask" "F.Paste") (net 12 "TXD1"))
  (pad "22" smd rect (at -0.85 7 90) (size 0.8 0.4) (layers "F.Cu" "F.Mask" "F.Paste") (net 13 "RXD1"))
  (pad "23" smd rect (at 0 7 90) (size 0.8 0.4) (layers "F.Cu" "F.Mask" "F.Paste") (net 18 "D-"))
  (pad "24" smd rect (at 0.85 7 90) (size 0.8 0.4) (layers "F.Cu" "F.Mask" "F.Paste") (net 17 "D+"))
  (pad "25" smd rect (at 1.7 7 90) (size 0.8 0.4) (layers "F.Cu" "F.Mask" "F.Paste") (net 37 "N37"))
  (pad "26" smd rect (at 2.55 7 90) (size 0.8 0.4) (layers "F.Cu" "F.Mask" "F.Paste") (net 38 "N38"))
  (pad "27" smd rect (at 3.4 7 90) (size 0.8 0.4) (layers "F.Cu" "F.Mask" "F.Paste") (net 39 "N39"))
  (pad "28" smd rect (at 4.25 7 90) (size 0.8 0.4) (layers "F.Cu" "F.Mask" "F.Paste") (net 30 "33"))
  (pad "29" smd rect (at 5.1 7 90) (size 0.8 0.4) (layers "F.Cu" "F.Mask" "F.Paste") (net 31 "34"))
  (pad "30" smd rect (at 5.95 7 90) (size 0.8 0.4) (layers "F.Cu" "F.Mask" "F.Paste") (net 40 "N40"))
  (pad "31" smd rect (at 7 5.95) (size 0.8 0.4) (layers "F.Cu" "F.Mask" "F.Paste") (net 32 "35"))
  (pad "32" smd rect (at 7 5.1) (size 0.8 0.4) (layers "F.Cu" "F.Mask" "F.Paste") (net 33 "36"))
  (pad "33" smd rect (at 7 4.25) (size 0.8 0.4) (layers "F.Cu" "F.Mask" "F.Paste") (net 34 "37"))
  (pad "34" smd rect (at 7 3.4) (size 0.8 0.4) (layers "F.Cu" "F.Mask" "F.Paste") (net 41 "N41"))
  (pad "35" smd rect (at 7 2.55) (size 0.8 0.4) (layers "F.Cu" "F.Mask" "F.Paste") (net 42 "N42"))
  (pad "36" smd rect (at 7 1.7) (size 0.8 0.4) (layers "F.Cu" "F.Mask" "F.Paste") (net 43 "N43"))
  (pad "37" smd rect (at 7 0.85) (size 0.8 0.4) (layers "F.Cu" "F.Mask" "F.Paste") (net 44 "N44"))
  (pad "38" smd rect (at 7 0) (size 0.8 0.4) (layers "F.Cu" "F.Mask" "F.Paste") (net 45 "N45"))
  (pad "39" smd rect (at 7 -0.85) (size 0.8 0.4) (layers "F.Cu" "F.Mask" "F.Paste") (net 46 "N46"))
  (pad "40" smd rect (at 7 -1.7) (size 0.8 0.4) (layers "F.Cu" "F.Mask" "F.Paste") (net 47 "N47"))
  (pad "41" smd rect (at 7 -2.55) (size 0.8 0.4) (layers "F.Cu" "F.Mask" "F.Paste") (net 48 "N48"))
  (pad "42" smd rect (at 7 -3.4) (size 0.8 0.4) (layers "F.Cu" "F.Mask" "F.Paste") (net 3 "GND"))
  (pad "43" smd rect (at 7 -4.25) (size 0.8 0.4) (layers "F.Cu" "F.Mask" "F.Paste") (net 3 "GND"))
  (pad "44" smd rect (at 7 -5.1) (size 0.8 0.4) (layers "F.Cu" "F.Mask" "F.Paste") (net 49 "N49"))
  (pad "45" smd rect (at 7 -5.95) (size 0.8 0.4) (layers "F.Cu" "F.Mask" "F.Paste") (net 4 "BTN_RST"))
  (pad "46" smd rect (at 5.95 -7 90) (size 0.8 0.4) (layers "F.Cu" "F.Mask" "F.Paste") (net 3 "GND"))
  (pad "47" smd rect (at 5.1 -7 90) (size 0.8 0.4) (layers "F.Cu" "F.Mask" "F.Paste") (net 3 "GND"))
  (pad "48" smd rect (at 4.25 -7 90) (size 0.8 0.4) (layers "F.Cu" "F.Mask" "F.Paste") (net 3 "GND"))
  (pad "49" smd rect (at 3.4 -7 90) (size 0.8 0.4) (layers "F.Cu" "F.Mask" "F.Paste") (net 3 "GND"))
  (pad "50" smd rect (at 2.55 -7 90) (size 0.8 0.4) (layers "F.Cu" "F.Mask" "F.Paste") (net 3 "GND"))
  (pad "51" smd rect (at 1.7 -7 90) (size 0.8 0.4) (layers "F.Cu" "F.Mask" "F.Paste") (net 3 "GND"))
  (pad "52" smd rect (at 0.85 -7 90) (size 0.8 0.4) (layers "F.Cu" "F.Mask" "F.Paste") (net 3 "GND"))
  (pad "53" smd rect (at 0 -7 90) (size 0.8 0.4) (layers "F.Cu" "F.Mask" "F.Paste") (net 3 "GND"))
  (pad "54" smd rect (at -0.85 -7 90) (size 0.8 0.4) (layers "F.Cu" "F.Mask" "F.Paste") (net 3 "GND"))
  (pad "55" smd rect (at -1.7 -7 90) (size 0.8 0.4) (layers "F.Cu" "F.Mask" "F.Paste") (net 3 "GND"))
  (pad "56" smd rect (at -2.55 -7 90) (size 0.8 0.4) (layers "F.Cu" "F.Mask" "F.Paste") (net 3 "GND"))
  (pad "57" smd rect (at -3.4 -7 90) (size 0.8 0.4) (layers "F.Cu" "F.Mask" "F.Paste") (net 3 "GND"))
  (pad "58" smd rect (at -4.25 -7 90) (size 0.8 0.4) (layers "F.Cu" "F.Mask" "F.Paste") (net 3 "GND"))
  (pad "59" smd rect (at -5.1 -7 90) (size 0.8 0.4) (layers "F.Cu" "F.Mask" "F.Paste") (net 3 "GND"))
  (pad "60" smd rect (at -5.95 -7 90) (size 0.8 0.4) (layers "F.Cu" "F.Mask" "F.Paste") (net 3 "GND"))
  (pad "61" smd roundrect (at -1.65 -1.65) (size 1.2 1.2) (layers "F.Cu" "F.Mask" "F.Paste") (roundrect_rratio 0) (chamfer_ratio 0.33)
   (chamfer top_left) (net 3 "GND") (zone_connect 2))
  (pad "61" smd rect (at -1.65 0) (size 1.2 1.2) (layers "F.Cu" "F.Mask" "F.Paste") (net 3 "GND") (zone_connect 2))
  (pad "61" smd rect (at -1.65 1.65) (size 1.2 1.2) (layers "F.Cu" "F.Mask" "F.Paste") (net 3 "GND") (zone_connect 2))
  (pad "61" smd rect (at 0 -1.65) (size 1.2 1.2) (layers "F.Cu" "F.Mask" "F.Paste") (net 3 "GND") (zone_connect 2))
  (pad "61" smd rect (at 0 0) (size 1.2 1.2) (layers "F.Cu" "F.Mask" "F.Paste") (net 3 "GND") (zone_connect 2))
  (pad "61" smd rect (at 0 1.65) (size 1.2 1.2) (layers "F.Cu" "F.Mask" "F.Paste") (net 3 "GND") (zone_connect 2))
  (pad "61" smd rect (at 1.65 -1.65) (size 1.2 1.2) (layers "F.Cu" "F.Mask" "F.Paste") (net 3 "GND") (zone_connect 2))
  (pad "61" smd rect (at 1.65 0) (size 1.2 1.2) (layers "F.Cu" "F.Mask" "F.Paste") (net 3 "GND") (zone_connect 2))
  (pad "61" smd rect (at 1.65 1.65) (size 1.2 1.2) (layers "F.Cu" "F.Mask" "F.Paste") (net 3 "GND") (zone_connect 2))
  (pad "62" smd rect (at -7 -7) (size 0.8 0.8) (layers "F.Cu" "F.Mask" "F.Paste") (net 3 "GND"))
  (pad "63" smd rect (at -7 7) (size 0.8 0.8) (layers "F.Cu" "F.Mask" "F.Paste") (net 3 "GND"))
  (pad "64" smd rect (at 7 7) (size 0.8 0.8) (layers "F.Cu" "F.Mask" "F.Paste") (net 3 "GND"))
  (pad "65" smd rect (at 7 -7) (size 0.8 0.8) (layers "F.Cu" "F.Mask" "F.Paste") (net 3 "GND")))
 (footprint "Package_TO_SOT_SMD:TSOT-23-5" (layer "F.Cu") (at 146.05 83.5 180)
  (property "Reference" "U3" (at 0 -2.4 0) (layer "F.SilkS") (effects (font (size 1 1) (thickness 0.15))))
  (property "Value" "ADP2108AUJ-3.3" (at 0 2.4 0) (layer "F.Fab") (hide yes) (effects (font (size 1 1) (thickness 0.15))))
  (fp_line (start 0 1.56) (end 0.8 1.56) (stroke (width 0.12) (type solid)) (layer "F.SilkS"))
  (fp_line (start 0 1.56) (end -0.8 1.56) (stroke (width 0.12) (type solid)) (layer "F.SilkS"))
  (fp_line (start 0 -1.56) (end 0.8 -1.56) (stroke (width 0.12) (type solid)) (layer "F.SilkS"))
  (fp_line (start 0 -1.56) (end -0.8 -1.56) (stroke (width 0.12) (type solid)) (layer "F.SilkS"))
  (fp_poly (pts (xy -1.3 -1.51) (xy -1.54 -1.84) (xy -1.06 -1.84)) (stroke (width 0.12) (type solid)) (fill yes) (layer "F.SilkS"))
  (pad "1" smd roundrect (at -1.1375 -0.95 180) (size 1.325 0.6) (layers "F.Cu" "F.Mask" "F.Paste") (roundrect_rratio 0.25)
   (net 14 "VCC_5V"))
  (pad "2" smd roundrect (at -1.1375 0 180) (size 1.325 0.6) (layers "F.Cu" "F.Mask" "F.Paste") (roundrect_rratio 0.25) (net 3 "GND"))
  (pad "3" smd roundrect (at -1.1375 0.95 180) (size 1.325 0.6) (layers "F.Cu" "F.Mask" "F.Paste") (roundrect_rratio 0.25) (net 14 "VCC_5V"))
  (pad "4" smd roundrect (at 1.1375 0.95 180) (size 1.325 0.6) (layers "F.Cu" "F.Mask" "F.Paste") (roundrect_rratio 0.25) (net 1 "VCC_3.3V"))
  (pad "5" smd roundrect (at 1.1375 -0.95 180) (size 1.325 0.6) (layers "F.Cu" "F.Mask" "F.Paste") (roundrect_rratio 0.25) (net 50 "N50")))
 (gr_rect (start 137.922 64.262) (end 164.338 105.918) (stroke (width 0.05) (type default)) (fill no) (layer "Edge.Cuts"))
 (via (at 146.05 71.374) (size 0.6) (drill 0.3) (layers "F.Cu" "B.Cu") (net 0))
 (via (at 146.05 70.612) (size 0.6) (drill 0.3) (layers "F.Cu" "B.Cu") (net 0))
 (via (at 146.05 75.946) (size 0.6) (drill 0.3) (layers "F.Cu" "B.Cu") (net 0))
 (via (at 146.05 72.136) (size 0.6) (drill 0.3) (layers "F.Cu" "B.Cu") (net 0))
 (via (at 146.05 74.422) (size 0.6) (drill 0.3) (layers "F.Cu" "B.Cu") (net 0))
 (via (at 146.05 75.184) (size 0.6) (drill 0.3) (layers "F.Cu" "B.Cu") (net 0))
 (via (at 146.05 76.708) (size 0.6) (drill 0.3) (layers "F.Cu" "B.Cu") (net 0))
 (via (at 146.05 69.85) (size 0.6) (drill 0.3) (layers "F.Cu" "B.Cu") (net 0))
 (via (at 146.05 73.66) (size 0.6) (drill 0.3) (layers "F.Cu" "B.Cu") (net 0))
 (via (at 146.05 72.898) (size 0.6) (drill 0.3) (layers "F.Cu" "B.Cu") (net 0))
 (segment (start 160.54 66.04) (end 162.56 66.04) (width 0.2) (layer "F.Cu") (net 3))
 (segment (start 162.12 68.14) (end 162.56 68.58) (width 0.2) (layer "F.Cu") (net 3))
 (segment (start 144.13 67.29) (end 144.13 66.44) (width 0.2) (layer "F.Cu") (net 3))
 (segment (start 162.56 68.58) (end 160.58 68.58) (width 0.2) (layer "F.Cu") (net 3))
 (segment (start 139.7 66.04) (end 142.04 66.04) (width 0.2) (layer "F.Cu") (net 3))
 (segment (start 144.13 65.39) (end 158.13 65.39) (width 0.2) (layer "F.Cu") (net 3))
 (segment (start 144.13 66.44) (end 144.13 65.39) (width 0.2) (layer "F.Cu") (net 3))
 (segment (start 144.13 66.44) (end 142.44 66.44) (width 0.2) (layer "F.Cu") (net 3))
 (segment (start 160.14 68.14) (end 158.13 68.14) (width 0.2) (layer "F.Cu") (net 3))
 (segment (start 158.13 68.99) (end 158.13 68.14) (width 0.2) (layer "F.Cu") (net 3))
 (segment (start 162.56 66.04) (end 162.56 68.58) (width 0.2) (layer "F.Cu") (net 3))
 (segment (start 160.58 68.58) (end 160.14 68.14) (width 0.2) (layer "F.Cu") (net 3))
 (segment (start 158.13 65.39) (end 159.89 65.39) (width 0.2) (layer "F.Cu") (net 3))
 (segment (start 142.44 66.44) (end 142.04 66.04) (width 0.2) (layer "F.Cu") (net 3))
 (segment (start 159.89 65.39) (end 160.54 66.04) (width 0.2) (layer "F.Cu") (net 3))
 (segment (start 139.7 68.58) (end 140.14 68.14) (width 0.2) (layer "F.Cu") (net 1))
 (segment (start 140.14 68.14) (end 144.13 68.14) (width 0.2) (layer "F.Cu") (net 1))
 (segment (start 141.83 68.99) (end 144.13 68.99) (width 0.2) (layer "F.Cu") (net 2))
 (segment (start 139.7 71.12) (end 141.83 68.99) (width 0.2) (layer "F.Cu") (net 2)))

